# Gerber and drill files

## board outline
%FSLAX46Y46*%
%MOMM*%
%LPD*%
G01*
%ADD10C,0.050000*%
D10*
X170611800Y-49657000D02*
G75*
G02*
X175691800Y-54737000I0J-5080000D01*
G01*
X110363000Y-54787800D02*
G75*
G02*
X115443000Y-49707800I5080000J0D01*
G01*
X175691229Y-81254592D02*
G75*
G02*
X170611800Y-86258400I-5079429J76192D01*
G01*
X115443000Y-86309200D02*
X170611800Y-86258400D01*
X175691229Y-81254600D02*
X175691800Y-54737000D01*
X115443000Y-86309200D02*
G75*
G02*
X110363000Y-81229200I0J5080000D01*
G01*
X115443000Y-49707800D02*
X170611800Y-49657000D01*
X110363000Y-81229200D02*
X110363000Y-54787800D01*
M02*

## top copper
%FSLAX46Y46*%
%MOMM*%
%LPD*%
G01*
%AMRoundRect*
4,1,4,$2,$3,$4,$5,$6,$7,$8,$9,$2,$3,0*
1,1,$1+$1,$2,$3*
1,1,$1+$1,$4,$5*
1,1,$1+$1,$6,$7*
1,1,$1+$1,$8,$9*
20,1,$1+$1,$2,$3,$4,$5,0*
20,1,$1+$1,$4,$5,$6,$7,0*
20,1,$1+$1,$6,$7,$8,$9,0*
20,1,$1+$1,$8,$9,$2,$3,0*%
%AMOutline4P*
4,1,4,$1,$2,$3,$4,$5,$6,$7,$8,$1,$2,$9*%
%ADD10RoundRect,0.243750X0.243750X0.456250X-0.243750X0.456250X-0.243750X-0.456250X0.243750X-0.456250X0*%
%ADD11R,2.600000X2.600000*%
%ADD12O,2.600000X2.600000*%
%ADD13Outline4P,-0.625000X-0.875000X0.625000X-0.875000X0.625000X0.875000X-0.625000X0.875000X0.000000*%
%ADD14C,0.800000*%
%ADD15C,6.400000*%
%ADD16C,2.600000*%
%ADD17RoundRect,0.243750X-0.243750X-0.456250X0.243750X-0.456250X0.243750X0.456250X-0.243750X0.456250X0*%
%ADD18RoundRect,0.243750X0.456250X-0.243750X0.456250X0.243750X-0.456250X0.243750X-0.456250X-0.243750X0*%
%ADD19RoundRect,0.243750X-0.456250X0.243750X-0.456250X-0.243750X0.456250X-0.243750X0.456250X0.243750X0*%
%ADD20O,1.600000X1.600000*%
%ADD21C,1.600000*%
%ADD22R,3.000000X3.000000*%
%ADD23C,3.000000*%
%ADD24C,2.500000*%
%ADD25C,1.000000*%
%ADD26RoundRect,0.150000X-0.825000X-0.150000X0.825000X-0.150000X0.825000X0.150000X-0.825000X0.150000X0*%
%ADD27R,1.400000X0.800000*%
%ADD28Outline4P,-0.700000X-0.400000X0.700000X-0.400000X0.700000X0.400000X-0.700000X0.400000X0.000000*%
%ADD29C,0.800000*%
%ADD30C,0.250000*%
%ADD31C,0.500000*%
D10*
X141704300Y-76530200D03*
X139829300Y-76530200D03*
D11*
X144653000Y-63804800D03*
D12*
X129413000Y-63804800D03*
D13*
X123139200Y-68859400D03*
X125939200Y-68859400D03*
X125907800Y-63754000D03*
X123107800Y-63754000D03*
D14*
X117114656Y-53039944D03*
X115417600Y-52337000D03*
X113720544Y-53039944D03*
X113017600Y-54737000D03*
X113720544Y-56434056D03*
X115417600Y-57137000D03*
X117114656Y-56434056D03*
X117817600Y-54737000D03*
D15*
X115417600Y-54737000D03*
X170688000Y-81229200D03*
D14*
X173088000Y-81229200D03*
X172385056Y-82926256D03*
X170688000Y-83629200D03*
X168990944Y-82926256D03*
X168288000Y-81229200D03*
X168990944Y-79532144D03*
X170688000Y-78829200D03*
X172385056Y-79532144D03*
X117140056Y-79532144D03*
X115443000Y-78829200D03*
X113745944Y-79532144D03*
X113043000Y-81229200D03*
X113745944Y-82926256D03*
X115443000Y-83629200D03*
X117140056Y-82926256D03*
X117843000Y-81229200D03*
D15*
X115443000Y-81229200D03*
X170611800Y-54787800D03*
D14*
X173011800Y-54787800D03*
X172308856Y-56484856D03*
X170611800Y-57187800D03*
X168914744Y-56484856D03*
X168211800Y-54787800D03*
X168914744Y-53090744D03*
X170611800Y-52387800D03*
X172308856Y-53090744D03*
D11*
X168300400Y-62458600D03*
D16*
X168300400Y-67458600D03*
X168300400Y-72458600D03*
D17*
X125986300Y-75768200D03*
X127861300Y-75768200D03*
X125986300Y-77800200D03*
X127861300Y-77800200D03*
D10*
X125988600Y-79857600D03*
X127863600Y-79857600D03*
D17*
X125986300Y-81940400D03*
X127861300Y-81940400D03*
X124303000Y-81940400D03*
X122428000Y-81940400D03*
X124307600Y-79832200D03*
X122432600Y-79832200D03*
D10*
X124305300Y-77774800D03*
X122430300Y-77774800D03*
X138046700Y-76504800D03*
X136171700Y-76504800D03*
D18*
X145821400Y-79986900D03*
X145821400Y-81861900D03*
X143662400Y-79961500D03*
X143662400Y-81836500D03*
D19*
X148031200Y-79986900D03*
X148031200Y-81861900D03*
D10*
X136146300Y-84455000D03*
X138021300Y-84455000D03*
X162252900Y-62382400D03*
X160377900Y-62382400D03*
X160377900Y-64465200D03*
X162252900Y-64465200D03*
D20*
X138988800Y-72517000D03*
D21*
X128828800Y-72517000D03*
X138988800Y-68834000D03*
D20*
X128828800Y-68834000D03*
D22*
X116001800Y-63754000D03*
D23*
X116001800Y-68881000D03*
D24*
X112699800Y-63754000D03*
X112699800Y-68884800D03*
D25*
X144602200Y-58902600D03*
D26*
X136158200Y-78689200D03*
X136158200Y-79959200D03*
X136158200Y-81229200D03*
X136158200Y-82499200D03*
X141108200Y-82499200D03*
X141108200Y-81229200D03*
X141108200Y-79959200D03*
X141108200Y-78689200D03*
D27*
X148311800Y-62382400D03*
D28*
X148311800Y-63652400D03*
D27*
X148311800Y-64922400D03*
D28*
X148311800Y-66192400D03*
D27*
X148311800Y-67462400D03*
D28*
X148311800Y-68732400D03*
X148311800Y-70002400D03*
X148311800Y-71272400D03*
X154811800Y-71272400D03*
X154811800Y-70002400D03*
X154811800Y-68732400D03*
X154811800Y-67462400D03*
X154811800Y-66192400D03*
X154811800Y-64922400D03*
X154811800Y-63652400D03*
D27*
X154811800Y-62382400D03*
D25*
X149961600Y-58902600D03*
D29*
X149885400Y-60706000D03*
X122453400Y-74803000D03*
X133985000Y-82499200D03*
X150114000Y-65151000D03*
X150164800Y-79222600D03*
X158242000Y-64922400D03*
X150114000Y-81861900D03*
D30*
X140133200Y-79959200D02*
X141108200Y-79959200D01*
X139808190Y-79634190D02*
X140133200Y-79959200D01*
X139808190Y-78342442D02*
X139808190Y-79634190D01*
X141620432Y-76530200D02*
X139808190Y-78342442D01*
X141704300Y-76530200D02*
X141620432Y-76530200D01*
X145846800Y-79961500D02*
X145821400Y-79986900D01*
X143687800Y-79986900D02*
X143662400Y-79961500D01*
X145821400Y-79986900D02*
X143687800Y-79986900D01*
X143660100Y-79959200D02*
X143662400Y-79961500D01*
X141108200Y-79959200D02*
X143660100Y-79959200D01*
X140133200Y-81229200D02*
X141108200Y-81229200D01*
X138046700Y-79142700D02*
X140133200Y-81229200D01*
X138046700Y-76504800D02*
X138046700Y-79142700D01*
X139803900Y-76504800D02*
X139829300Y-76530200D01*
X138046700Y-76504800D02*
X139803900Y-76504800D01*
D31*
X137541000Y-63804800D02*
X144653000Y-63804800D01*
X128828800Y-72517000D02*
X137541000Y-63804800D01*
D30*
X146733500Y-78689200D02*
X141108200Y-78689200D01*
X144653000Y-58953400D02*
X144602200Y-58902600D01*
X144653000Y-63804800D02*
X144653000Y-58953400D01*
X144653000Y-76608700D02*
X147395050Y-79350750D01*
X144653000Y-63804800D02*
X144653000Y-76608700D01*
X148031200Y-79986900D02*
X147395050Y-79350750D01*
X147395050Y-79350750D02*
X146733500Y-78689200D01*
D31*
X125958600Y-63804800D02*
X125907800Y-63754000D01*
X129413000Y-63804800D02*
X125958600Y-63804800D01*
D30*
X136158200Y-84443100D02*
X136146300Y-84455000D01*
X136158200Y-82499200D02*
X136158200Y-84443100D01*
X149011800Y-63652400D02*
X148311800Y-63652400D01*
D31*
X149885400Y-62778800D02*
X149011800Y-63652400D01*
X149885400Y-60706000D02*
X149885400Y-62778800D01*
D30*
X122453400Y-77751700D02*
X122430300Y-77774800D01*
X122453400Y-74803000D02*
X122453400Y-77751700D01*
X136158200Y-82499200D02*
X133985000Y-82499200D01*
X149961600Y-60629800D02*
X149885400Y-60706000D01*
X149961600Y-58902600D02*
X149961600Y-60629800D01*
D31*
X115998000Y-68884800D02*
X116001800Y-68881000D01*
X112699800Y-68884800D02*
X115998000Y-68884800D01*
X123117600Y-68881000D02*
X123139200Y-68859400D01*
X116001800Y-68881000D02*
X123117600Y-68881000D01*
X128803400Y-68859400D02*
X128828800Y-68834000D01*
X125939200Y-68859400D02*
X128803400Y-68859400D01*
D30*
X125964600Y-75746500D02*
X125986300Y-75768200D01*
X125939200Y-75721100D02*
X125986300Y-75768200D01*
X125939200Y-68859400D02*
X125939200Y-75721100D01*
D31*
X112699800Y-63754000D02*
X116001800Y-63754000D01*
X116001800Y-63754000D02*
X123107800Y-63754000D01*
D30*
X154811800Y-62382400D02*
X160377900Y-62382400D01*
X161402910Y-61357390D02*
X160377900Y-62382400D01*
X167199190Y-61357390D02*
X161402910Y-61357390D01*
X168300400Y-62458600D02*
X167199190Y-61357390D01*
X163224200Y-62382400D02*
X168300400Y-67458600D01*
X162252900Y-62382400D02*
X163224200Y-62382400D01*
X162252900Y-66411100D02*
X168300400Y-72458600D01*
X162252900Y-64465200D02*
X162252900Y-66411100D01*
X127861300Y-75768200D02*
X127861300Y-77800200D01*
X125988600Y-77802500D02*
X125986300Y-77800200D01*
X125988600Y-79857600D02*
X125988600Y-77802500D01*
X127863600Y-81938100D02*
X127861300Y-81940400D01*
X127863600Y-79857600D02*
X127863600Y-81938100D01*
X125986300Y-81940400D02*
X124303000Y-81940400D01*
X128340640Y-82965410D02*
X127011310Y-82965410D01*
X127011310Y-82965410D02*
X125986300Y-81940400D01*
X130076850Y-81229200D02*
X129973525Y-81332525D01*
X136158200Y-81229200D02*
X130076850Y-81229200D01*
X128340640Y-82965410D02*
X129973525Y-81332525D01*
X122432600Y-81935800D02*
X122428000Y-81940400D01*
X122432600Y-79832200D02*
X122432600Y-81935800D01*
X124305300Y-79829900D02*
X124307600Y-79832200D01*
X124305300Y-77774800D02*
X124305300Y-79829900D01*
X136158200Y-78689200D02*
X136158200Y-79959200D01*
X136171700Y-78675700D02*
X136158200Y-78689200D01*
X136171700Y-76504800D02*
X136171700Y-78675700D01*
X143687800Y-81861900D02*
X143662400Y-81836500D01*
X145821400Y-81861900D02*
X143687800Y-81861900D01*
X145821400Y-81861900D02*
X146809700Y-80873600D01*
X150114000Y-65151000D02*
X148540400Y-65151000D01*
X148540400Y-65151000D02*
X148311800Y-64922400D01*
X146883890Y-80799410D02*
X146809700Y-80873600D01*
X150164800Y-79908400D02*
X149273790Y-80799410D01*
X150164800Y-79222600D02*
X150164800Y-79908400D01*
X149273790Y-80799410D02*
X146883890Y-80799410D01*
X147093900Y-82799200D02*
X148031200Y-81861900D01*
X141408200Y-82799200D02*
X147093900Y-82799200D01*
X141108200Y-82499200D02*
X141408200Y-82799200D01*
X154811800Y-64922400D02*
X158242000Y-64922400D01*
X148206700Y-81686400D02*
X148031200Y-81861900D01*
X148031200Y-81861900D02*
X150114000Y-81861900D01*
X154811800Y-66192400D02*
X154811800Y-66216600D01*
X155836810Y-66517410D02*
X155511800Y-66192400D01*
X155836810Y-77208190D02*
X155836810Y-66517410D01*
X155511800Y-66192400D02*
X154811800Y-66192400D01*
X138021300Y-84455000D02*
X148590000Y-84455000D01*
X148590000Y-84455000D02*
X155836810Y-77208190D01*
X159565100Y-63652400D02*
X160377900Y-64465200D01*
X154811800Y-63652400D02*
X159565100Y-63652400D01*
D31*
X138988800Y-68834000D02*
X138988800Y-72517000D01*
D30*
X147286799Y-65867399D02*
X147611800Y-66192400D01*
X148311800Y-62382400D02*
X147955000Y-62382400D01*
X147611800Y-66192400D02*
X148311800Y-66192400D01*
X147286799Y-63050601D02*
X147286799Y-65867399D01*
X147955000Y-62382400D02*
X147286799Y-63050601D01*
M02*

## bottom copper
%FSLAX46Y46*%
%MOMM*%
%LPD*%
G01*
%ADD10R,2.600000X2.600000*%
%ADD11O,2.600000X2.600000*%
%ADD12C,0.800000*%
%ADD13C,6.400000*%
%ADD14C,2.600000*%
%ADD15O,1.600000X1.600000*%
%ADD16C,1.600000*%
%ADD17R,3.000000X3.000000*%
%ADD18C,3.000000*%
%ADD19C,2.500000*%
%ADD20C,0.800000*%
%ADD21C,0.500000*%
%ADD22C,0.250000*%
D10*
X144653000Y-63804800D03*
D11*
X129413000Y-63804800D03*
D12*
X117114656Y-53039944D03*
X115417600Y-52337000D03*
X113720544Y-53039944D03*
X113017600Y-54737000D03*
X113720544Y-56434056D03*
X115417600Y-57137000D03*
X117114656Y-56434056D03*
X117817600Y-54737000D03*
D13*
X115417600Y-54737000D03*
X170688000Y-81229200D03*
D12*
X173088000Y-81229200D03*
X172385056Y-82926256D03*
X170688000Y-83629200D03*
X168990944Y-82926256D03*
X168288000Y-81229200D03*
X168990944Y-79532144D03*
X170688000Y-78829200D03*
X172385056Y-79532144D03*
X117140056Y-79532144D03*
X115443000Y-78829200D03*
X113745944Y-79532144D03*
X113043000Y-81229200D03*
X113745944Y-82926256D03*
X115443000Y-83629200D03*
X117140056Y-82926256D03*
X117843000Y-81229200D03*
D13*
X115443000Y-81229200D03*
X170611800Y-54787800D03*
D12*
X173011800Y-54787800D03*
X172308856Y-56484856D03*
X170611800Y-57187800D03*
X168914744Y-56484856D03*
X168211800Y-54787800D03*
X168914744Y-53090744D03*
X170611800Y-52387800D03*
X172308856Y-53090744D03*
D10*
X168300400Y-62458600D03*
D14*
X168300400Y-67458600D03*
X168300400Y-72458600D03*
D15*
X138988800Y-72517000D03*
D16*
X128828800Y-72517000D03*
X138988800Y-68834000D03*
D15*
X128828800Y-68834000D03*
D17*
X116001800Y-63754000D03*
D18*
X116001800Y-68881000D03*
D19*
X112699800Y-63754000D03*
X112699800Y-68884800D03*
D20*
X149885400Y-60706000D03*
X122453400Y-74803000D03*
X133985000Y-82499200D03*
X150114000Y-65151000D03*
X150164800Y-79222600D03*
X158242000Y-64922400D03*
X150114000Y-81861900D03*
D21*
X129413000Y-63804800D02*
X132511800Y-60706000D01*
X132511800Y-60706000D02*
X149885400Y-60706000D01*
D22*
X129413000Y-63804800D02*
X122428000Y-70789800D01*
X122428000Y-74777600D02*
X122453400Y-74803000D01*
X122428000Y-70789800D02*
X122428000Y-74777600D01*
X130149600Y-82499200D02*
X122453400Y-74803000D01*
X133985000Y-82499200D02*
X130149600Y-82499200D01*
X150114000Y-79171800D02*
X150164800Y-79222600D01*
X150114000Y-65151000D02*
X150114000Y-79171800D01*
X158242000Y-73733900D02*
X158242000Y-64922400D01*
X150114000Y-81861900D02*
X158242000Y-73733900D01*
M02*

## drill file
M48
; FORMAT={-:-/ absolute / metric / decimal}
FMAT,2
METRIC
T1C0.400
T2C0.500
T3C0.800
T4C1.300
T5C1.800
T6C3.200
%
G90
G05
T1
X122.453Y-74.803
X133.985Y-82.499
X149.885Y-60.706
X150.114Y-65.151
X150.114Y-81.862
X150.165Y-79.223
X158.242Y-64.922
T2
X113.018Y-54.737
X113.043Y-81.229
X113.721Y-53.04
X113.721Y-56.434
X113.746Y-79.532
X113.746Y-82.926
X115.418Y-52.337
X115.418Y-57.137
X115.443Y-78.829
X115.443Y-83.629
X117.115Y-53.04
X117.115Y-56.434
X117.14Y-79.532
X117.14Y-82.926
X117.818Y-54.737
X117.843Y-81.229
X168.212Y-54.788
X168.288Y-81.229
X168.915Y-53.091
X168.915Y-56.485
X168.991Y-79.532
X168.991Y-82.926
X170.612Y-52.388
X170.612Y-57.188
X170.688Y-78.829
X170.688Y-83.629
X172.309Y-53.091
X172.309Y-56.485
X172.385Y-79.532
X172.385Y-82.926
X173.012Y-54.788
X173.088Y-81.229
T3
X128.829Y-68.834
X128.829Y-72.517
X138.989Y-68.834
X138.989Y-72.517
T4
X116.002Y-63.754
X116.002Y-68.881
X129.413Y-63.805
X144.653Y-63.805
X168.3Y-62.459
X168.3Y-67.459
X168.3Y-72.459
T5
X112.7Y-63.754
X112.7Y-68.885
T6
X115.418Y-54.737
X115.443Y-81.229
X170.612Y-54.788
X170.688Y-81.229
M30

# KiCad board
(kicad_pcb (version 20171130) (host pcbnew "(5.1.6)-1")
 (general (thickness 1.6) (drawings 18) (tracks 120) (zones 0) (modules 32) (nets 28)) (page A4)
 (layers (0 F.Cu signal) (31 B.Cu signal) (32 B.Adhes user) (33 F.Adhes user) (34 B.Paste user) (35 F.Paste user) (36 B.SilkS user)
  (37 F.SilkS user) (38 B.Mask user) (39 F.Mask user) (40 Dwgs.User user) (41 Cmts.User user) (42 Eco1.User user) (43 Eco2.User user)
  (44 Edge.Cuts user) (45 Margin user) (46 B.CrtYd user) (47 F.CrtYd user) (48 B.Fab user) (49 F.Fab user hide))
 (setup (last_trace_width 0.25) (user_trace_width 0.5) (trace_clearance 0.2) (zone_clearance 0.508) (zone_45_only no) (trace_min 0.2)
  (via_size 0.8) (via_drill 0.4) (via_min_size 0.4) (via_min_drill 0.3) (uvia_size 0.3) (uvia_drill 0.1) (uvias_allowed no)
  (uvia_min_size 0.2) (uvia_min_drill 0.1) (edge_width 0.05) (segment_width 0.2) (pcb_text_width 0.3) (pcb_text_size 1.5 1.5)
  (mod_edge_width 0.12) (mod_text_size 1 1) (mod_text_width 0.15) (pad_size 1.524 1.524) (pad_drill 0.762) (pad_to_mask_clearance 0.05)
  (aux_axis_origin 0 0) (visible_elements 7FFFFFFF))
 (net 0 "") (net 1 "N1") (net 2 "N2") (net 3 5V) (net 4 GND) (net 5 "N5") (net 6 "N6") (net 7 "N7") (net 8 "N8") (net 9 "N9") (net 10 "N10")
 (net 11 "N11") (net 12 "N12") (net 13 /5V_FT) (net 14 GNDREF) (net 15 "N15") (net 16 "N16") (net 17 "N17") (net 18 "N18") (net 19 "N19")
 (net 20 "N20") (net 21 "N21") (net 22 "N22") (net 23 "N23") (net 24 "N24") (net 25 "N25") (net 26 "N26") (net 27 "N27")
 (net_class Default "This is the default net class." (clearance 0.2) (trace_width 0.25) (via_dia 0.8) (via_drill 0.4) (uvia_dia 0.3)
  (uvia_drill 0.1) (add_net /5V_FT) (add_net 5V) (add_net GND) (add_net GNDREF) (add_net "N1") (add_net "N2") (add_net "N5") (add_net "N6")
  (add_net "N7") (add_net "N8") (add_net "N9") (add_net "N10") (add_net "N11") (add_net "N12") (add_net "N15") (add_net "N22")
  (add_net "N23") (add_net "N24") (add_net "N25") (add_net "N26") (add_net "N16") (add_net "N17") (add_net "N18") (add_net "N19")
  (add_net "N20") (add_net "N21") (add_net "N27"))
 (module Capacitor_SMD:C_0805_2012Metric (layer F.Cu) (at 140.7668 76.5302 180)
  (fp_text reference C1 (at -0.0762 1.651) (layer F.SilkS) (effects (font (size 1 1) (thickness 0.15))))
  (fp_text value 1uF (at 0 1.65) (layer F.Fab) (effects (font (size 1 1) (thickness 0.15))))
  (pad 1 smd roundrect (at -0.9375 0 180) (size 0.975 1.4) (layers F.Cu F.Paste F.Mask) (roundrect_rratio 0.25) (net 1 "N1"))
  (pad 2 smd roundrect (at 0.9375 0 180) (size 0.975 1.4) (layers F.Cu F.Paste F.Mask) (roundrect_rratio 0.25) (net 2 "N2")))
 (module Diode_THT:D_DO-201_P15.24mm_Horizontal (layer F.Cu) (at 144.653 63.8048 180)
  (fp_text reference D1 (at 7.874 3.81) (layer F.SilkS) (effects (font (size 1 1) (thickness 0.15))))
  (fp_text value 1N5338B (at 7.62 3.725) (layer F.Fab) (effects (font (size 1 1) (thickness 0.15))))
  (pad 1 thru_hole rect (at 0 0 180) (size 2.6 2.6) (drill 1.3) (layers *.Cu *.Mask) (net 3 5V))
  (pad 2 thru_hole oval (at 15.24 0 180) (size 2.6 2.6) (drill 1.3) (layers *.Cu *.Mask) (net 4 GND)))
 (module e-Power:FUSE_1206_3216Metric (layer F.Cu) (at 124.5392 68.8594)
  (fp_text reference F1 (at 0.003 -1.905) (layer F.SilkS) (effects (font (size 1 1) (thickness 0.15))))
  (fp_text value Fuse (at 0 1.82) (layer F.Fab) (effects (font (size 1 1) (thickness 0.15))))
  (pad 1 smd trapezoid (at -1.4 0) (size 1.25 1.75) (layers F.Cu F.Paste F.Mask) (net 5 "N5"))
  (pad 2 smd trapezoid (at 1.4 0) (size 1.25 1.75) (layers F.Cu F.Paste F.Mask) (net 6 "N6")))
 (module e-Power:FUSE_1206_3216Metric (layer F.Cu) (at 124.5078 63.754)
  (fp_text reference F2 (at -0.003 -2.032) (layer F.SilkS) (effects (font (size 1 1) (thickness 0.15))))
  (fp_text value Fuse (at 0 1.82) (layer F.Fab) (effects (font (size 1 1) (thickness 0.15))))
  (pad 2 smd trapezoid (at 1.4 0) (size 1.25 1.75) (layers F.Cu F.Paste F.Mask) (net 4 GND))
  (pad 1 smd trapezoid (at -1.4 0) (size 1.25 1.75) (layers F.Cu F.Paste F.Mask) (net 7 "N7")))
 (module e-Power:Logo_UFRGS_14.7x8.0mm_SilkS (layer F.Cu) (at 159.3596 81.2546)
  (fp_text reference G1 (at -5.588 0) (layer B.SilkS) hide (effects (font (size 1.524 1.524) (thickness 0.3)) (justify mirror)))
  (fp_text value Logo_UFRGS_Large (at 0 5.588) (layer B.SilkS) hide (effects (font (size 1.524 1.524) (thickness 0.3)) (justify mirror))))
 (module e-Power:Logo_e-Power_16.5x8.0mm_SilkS (layer F.Cu) (at 158.1912 54.7878)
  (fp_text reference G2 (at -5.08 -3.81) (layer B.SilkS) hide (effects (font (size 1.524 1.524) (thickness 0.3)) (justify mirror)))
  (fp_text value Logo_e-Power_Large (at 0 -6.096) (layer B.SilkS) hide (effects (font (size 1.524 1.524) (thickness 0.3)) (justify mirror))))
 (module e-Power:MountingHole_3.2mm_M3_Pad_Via (layer F.Cu) (at 115.4176 54.737)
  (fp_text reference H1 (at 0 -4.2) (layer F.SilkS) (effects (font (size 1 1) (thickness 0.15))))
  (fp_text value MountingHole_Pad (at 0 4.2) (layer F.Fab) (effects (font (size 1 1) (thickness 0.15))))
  (pad 1 thru_hole circle (at 1.697056 -1.697056) (size 0.8 0.8) (drill 0.5) (layers *.Cu *.Mask) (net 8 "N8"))
  (pad 1 thru_hole circle (at 0 -2.4) (size 0.8 0.8) (drill 0.5) (layers *.Cu *.Mask) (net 8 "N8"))
  (pad 1 thru_hole circle (at -1.697056 -1.697056) (size 0.8 0.8) (drill 0.5) (layers *.Cu *.Mask) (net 8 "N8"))
  (pad 1 thru_hole circle (at -2.4 0) (size 0.8 0.8) (drill 0.5) (layers *.Cu *.Mask) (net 8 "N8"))
  (pad 1 thru_hole circle (at -1.697056 1.697056) (size 0.8 0.8) (drill 0.5) (layers *.Cu *.Mask) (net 8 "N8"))
  (pad 1 thru_hole circle (at 0 2.4) (size 0.8 0.8) (drill 0.5) (layers *.Cu *.Mask) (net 8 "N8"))
  (pad 1 thru_hole circle (at 1.697056 1.697056) (size 0.8 0.8) (drill 0.5) (layers *.Cu *.Mask) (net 8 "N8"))
  (pad 1 thru_hole circle (at 2.4 0) (size 0.8 0.8) (drill 0.5) (layers *.Cu *.Mask) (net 8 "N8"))
  (pad 1 thru_hole circle (at 0 0) (size 6.4 6.4) (drill 3.2) (layers *.Cu *.Mask) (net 8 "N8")))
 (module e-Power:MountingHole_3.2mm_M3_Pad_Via (layer F.Cu) (at 170.688 81.2292)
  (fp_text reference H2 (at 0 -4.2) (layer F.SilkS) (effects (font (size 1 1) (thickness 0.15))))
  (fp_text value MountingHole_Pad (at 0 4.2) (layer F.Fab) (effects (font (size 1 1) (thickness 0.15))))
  (pad 1 thru_hole circle (at 0 0) (size 6.4 6.4) (drill 3.2) (layers *.Cu *.Mask) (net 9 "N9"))
  (pad 1 thru_hole circle (at 2.4 0) (size 0.8 0.8) (drill 0.5) (layers *.Cu *.Mask) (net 9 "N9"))
  (pad 1 thru_hole circle (at 1.697056 1.697056) (size 0.8 0.8) (drill 0.5) (layers *.Cu *.Mask) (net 9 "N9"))
  (pad 1 thru_hole circle (at 0 2.4) (size 0.8 0.8) (drill 0.5) (layers *.Cu *.Mask) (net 9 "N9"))
  (pad 1 thru_hole circle (at -1.697056 1.697056) (size 0.8 0.8) (drill 0.5) (layers *.Cu *.Mask) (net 9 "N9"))
  (pad 1 thru_hole circle (at -2.4 0) (size 0.8 0.8) (drill 0.5) (layers *.Cu *.Mask) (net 9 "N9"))
  (pad 1 thru_hole circle (at -1.697056 -1.697056) (size 0.8 0.8) (drill 0.5) (layers *.Cu *.Mask) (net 9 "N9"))
  (pad 1 thru_hole circle (at 0 -2.4) (size 0.8 0.8) (drill 0.5) (layers *.Cu *.Mask) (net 9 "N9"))
  (pad 1 thru_hole circle (at 1.697056 -1.697056) (size 0.8 0.8) (drill 0.5) (layers *.Cu *.Mask) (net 9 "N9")))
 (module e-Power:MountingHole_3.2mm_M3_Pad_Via (layer F.Cu) (at 115.443 81.2292)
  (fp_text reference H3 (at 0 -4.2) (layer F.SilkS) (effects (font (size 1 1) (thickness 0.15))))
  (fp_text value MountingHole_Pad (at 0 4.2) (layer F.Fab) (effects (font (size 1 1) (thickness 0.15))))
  (pad 1 thru_hole circle (at 1.697056 -1.697056) (size 0.8 0.8) (drill 0.5) (layers *.Cu *.Mask) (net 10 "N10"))
  (pad 1 thru_hole circle (at 0 -2.4) (size 0.8 0.8) (drill 0.5) (layers *.Cu *.Mask) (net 10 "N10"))
  (pad 1 thru_hole circle (at -1.697056 -1.697056) (size 0.8 0.8) (drill 0.5) (layers *.Cu *.Mask) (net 10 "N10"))
  (pad 1 thru_hole circle (at -2.4 0) (size 0.8 0.8) (drill 0.5) (layers *.Cu *.Mask) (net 10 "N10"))
  (pad 1 thru_hole circle (at -1.697056 1.697056) (size 0.8 0.8) (drill 0.5) (layers *.Cu *.Mask) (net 10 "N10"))
  (pad 1 thru_hole circle (at 0 2.4) (size 0.8 0.8) (drill 0.5) (layers *.Cu *.Mask) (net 10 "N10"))
  (pad 1 thru_hole circle (at 1.697056 1.697056) (size 0.8 0.8) (drill 0.5) (layers *.Cu *.Mask) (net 10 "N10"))
  (pad 1 thru_hole circle (at 2.4 0) (size 0.8 0.8) (drill 0.5) (layers *.Cu *.Mask) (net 10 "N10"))
  (pad 1 thru_hole circle (at 0 0) (size 6.4 6.4) (drill 3.2) (layers *.Cu *.Mask) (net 10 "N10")))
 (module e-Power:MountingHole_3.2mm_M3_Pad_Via (layer F.Cu) (at 170.6118 54.7878)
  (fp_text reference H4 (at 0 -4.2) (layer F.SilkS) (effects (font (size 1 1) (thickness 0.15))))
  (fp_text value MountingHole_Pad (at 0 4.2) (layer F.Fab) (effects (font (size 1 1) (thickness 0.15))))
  (pad 1 thru_hole circle (at 0 0) (size 6.4 6.4) (drill 3.2) (layers *.Cu *.Mask) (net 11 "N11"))
  (pad 1 thru_hole circle (at 2.4 0) (size 0.8 0.8) (drill 0.5) (layers *.Cu *.Mask) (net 11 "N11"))
  (pad 1 thru_hole circle (at 1.697056 1.697056) (size 0.8 0.8) (drill 0.5) (layers *.Cu *.Mask) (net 11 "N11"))
  (pad 1 thru_hole circle (at 0 2.4) (size 0.8 0.8) (drill 0.5) (layers *.Cu *.Mask) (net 11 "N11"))
  (pad 1 thru_hole circle (at -1.697056 1.697056) (size 0.8 0.8) (drill 0.5) (layers *.Cu *.Mask) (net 11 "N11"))
  (pad 1 thru_hole circle (at -2.4 0) (size 0.8 0.8) (drill 0.5) (layers *.Cu *.Mask) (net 11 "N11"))
  (pad 1 thru_hole circle (at -1.697056 -1.697056) (size 0.8 0.8) (drill 0.5) (layers *.Cu *.Mask) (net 11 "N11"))
  (pad 1 thru_hole circle (at 0 -2.4) (size 0.8 0.8) (drill 0.5) (layers *.Cu *.Mask) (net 11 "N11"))
  (pad 1 thru_hole circle (at 1.697056 -1.697056) (size 0.8 0.8) (drill 0.5) (layers *.Cu *.Mask) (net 11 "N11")))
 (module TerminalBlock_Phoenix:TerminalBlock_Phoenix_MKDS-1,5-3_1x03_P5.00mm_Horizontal (layer F.Cu) (at 168.3004 62.4586 270)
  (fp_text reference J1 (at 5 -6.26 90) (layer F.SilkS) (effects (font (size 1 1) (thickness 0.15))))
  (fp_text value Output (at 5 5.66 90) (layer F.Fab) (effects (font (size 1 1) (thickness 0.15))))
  (pad 1 thru_hole rect (at 0 0 270) (size 2.6 2.6) (drill 1.3) (layers *.Cu *.Mask) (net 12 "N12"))
  (pad 2 thru_hole circle (at 5 0 270) (size 2.6 2.6) (drill 1.3) (layers *.Cu *.Mask) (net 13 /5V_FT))
  (pad 3 thru_hole circle (at 10 0 270) (size 2.6 2.6) (drill 1.3) (layers *.Cu *.Mask) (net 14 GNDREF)))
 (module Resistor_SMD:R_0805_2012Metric (layer F.Cu) (at 126.9238 75.7682)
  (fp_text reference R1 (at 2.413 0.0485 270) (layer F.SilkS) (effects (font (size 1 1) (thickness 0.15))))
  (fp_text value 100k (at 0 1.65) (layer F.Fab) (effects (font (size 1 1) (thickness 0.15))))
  (pad 1 smd roundrect (at -0.9375 0) (size 0.975 1.4) (layers F.Cu F.Paste F.Mask) (roundrect_rratio 0.25) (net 6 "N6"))
  (pad 2 smd roundrect (at 0.9375 0) (size 0.975 1.4) (layers F.Cu F.Paste F.Mask) (roundrect_rratio 0.25) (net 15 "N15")))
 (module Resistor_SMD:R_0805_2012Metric (layer F.Cu) (at 126.9238 77.8002)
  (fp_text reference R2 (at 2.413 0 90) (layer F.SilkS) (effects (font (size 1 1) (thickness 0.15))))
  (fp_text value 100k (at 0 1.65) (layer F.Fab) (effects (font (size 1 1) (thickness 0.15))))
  (pad 1 smd roundrect (at -0.9375 0) (size 0.975 1.4) (layers F.Cu F.Paste F.Mask) (roundrect_rratio 0.25) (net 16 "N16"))
  (pad 2 smd roundrect (at 0.9375 0) (size 0.975 1.4) (layers F.Cu F.Paste F.Mask) (roundrect_rratio 0.25) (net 15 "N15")))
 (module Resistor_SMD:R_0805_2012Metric (layer F.Cu) (at 126.9261 79.8576 180)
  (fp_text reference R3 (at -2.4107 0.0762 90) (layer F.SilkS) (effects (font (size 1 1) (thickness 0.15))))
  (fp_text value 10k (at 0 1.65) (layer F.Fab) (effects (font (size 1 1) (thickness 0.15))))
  (pad 2 smd roundrect (at 0.9375 0 180) (size 0.975 1.4) (layers F.Cu F.Paste F.Mask) (roundrect_rratio 0.25) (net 16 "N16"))
  (pad 1 smd roundrect (at -0.9375 0 180) (size 0.975 1.4) (layers F.Cu F.Paste F.Mask) (roundrect_rratio 0.25) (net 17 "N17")))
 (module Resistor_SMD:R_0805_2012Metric (layer F.Cu) (at 126.9238 81.9404)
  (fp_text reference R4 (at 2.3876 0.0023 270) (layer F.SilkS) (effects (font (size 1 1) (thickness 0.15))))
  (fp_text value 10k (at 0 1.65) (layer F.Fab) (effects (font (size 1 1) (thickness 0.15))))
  (pad 1 smd roundrect (at -0.9375 0) (size 0.975 1.4) (layers F.Cu F.Paste F.Mask) (roundrect_rratio 0.25) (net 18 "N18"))
  (pad 2 smd roundrect (at 0.9375 0) (size 0.975 1.4) (layers F.Cu F.Paste F.Mask) (roundrect_rratio 0.25) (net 17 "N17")))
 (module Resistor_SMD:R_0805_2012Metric (layer F.Cu) (at 123.3655 81.9404)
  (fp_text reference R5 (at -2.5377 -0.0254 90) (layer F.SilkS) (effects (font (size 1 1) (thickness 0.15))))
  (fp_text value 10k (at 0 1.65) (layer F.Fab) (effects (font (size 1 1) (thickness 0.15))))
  (pad 2 smd roundrect (at 0.9375 0) (size 0.975 1.4) (layers F.Cu F.Paste F.Mask) (roundrect_rratio 0.25) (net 18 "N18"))
  (pad 1 smd roundrect (at -0.9375 0) (size 0.975 1.4) (layers F.Cu F.Paste F.Mask) (roundrect_rratio 0.25) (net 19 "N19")))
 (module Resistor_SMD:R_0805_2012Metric (layer F.Cu) (at 123.3701 79.8322)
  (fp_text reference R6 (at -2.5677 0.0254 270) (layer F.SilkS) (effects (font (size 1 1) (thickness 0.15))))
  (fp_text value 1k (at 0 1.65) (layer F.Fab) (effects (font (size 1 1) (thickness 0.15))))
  (pad 2 smd roundrect (at 0.9375 0) (size 0.975 1.4) (layers F.Cu F.Paste F.Mask) (roundrect_rratio 0.25) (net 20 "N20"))
  (pad 1 smd roundrect (at -0.9375 0) (size 0.975 1.4) (layers F.Cu F.Paste F.Mask) (roundrect_rratio 0.25) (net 19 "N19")))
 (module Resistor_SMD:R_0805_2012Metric (layer F.Cu) (at 123.3678 77.7748 180)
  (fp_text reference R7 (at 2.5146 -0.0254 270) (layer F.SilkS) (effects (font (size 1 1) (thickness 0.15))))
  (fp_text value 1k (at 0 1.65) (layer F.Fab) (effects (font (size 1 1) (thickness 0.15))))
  (pad 1 smd roundrect (at -0.9375 0 180) (size 0.975 1.4) (layers F.Cu F.Paste F.Mask) (roundrect_rratio 0.25) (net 20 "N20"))
  (pad 2 smd roundrect (at 0.9375 0 180) (size 0.975 1.4) (layers F.Cu F.Paste F.Mask) (roundrect_rratio 0.25) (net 4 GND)))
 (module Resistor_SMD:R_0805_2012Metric (layer F.Cu) (at 137.1092 76.5048 180)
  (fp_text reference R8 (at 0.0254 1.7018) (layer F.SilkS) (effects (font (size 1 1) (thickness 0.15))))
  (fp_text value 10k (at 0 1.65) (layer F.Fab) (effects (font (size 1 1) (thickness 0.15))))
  (pad 1 smd roundrect (at -0.9375 0 180) (size 0.975 1.4) (layers F.Cu F.Paste F.Mask) (roundrect_rratio 0.25) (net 2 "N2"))
  (pad 2 smd roundrect (at 0.9375 0 180) (size 0.975 1.4) (layers F.Cu F.Paste F.Mask) (roundrect_rratio 0.25) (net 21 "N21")))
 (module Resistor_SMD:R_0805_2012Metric (layer F.Cu) (at 145.8214 80.9244 90)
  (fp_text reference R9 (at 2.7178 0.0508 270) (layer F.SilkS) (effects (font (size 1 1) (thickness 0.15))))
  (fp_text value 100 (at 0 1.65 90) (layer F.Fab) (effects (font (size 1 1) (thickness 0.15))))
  (pad 2 smd roundrect (at 0.9375 0 90) (size 0.975 1.4) (layers F.Cu F.Paste F.Mask) (roundrect_rratio 0.25) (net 1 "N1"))
  (pad 1 smd roundrect (at -0.9375 0 90) (size 0.975 1.4) (layers F.Cu F.Paste F.Mask) (roundrect_rratio 0.25) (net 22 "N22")))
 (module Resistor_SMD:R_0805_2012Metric (layer F.Cu) (at 143.6624 80.899 90)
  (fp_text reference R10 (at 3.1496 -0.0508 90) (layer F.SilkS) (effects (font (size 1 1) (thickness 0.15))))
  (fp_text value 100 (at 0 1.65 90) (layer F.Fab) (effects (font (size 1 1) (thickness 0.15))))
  (pad 2 smd roundrect (at 0.9375 0 90) (size 0.975 1.4) (layers F.Cu F.Paste F.Mask) (roundrect_rratio 0.25) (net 1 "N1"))
  (pad 1 smd roundrect (at -0.9375 0 90) (size 0.975 1.4) (layers F.Cu F.Paste F.Mask) (roundrect_rratio 0.25) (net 22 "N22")))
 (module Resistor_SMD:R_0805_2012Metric (layer F.Cu) (at 148.0312 80.9244 270)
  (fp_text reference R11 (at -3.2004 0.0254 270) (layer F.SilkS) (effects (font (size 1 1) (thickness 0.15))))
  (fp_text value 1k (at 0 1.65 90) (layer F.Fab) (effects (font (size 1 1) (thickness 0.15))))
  (pad 1 smd roundrect (at -0.9375 0 270) (size 0.975 1.4) (layers F.Cu F.Paste F.Mask) (roundrect_rratio 0.25) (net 3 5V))
  (pad 2 smd roundrect (at 0.9375 0 270) (size 0.975 1.4) (layers F.Cu F.Paste F.Mask) (roundrect_rratio 0.25) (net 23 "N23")))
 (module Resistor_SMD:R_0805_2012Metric (layer F.Cu) (at 137.0838 84.455 180)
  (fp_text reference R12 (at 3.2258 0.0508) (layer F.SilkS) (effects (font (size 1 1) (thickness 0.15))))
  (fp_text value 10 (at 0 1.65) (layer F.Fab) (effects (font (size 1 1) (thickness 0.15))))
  (pad 2 smd roundrect (at 0.9375 0 180) (size 0.975 1.4) (layers F.Cu F.Paste F.Mask) (roundrect_rratio 0.25) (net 4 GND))
  (pad 1 smd roundrect (at -0.9375 0 180) (size 0.975 1.4) (layers F.Cu F.Paste F.Mask) (roundrect_rratio 0.25) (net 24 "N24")))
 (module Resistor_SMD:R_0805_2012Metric (layer F.Cu) (at 161.3154 62.3824 180)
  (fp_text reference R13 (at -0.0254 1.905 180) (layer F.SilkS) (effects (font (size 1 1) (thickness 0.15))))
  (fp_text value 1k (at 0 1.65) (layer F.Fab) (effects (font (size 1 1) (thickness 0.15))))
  (pad 1 smd roundrect (at -0.9375 0 180) (size 0.975 1.4) (layers F.Cu F.Paste F.Mask) (roundrect_rratio 0.25) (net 13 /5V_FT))
  (pad 2 smd roundrect (at 0.9375 0 180) (size 0.975 1.4) (layers F.Cu F.Paste F.Mask) (roundrect_rratio 0.25) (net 12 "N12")))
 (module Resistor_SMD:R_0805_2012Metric (layer F.Cu) (at 161.3154 64.4652 180)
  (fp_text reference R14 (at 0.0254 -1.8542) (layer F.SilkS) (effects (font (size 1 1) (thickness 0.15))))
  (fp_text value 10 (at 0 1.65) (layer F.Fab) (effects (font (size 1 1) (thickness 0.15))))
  (pad 2 smd roundrect (at 0.9375 0 180) (size 0.975 1.4) (layers F.Cu F.Paste F.Mask) (roundrect_rratio 0.25) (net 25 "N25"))
  (pad 1 smd roundrect (at -0.9375 0 180) (size 0.975 1.4) (layers F.Cu F.Paste F.Mask) (roundrect_rratio 0.25) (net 14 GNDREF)))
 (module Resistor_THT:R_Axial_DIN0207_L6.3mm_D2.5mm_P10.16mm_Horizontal (layer F.Cu) (at 128.8288 72.517)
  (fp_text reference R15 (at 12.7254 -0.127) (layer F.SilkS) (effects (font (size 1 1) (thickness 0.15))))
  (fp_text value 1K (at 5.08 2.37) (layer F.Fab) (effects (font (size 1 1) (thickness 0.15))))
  (pad 2 thru_hole oval (at 10.16 0) (size 1.6 1.6) (drill 0.8) (layers *.Cu *.Mask) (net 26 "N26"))
  (pad 1 thru_hole circle (at 0 0) (size 1.6 1.6) (drill 0.8) (layers *.Cu *.Mask) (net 3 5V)))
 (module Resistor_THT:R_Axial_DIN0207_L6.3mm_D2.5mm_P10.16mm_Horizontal (layer F.Cu) (at 138.9888 68.834 180)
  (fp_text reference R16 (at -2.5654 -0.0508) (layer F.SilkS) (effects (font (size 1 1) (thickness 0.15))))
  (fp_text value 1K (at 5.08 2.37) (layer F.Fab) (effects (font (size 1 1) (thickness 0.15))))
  (pad 1 thru_hole circle (at 0 0 180) (size 1.6 1.6) (drill 0.8) (layers *.Cu *.Mask) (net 26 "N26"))
  (pad 2 thru_hole oval (at 10.16 0 180) (size 1.6 1.6) (drill 0.8) (layers *.Cu *.Mask) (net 6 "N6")))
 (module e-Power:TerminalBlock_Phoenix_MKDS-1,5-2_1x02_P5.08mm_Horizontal (layer F.Cu) (at 116.0018 63.754 270)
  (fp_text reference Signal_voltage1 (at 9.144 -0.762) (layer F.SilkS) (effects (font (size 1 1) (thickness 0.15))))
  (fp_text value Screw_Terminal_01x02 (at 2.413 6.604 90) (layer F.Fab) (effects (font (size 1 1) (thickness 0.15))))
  (pad 1 thru_hole rect (at 0 0 270) (size 3 3) (drill 1.3) (layers *.Cu *.Mask) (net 7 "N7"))
  (pad 2 thru_hole circle (at 5.127 0 270) (size 3 3) (drill 1.3) (layers *.Cu *.Mask) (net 5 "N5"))
  (pad 1 thru_hole circle (at 0 3.302 270) (size 2.5 2.5) (drill 1.8) (layers *.Cu *.Mask) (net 7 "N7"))
  (pad 2 thru_hole circle (at 5.1308 3.302 270) (size 2.5 2.5) (drill 1.8) (layers *.Cu *.Mask) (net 5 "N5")))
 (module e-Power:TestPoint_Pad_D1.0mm (layer F.Cu) (at 144.6022 58.9026)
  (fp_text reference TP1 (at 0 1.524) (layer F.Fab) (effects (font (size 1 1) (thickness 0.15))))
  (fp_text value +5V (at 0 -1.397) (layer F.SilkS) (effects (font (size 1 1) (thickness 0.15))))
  (pad 1 smd circle (at 0 0) (size 1 1) (layers F.Cu F.Mask) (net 3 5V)))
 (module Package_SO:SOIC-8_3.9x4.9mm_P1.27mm (layer F.Cu) (at 138.6332 80.5942)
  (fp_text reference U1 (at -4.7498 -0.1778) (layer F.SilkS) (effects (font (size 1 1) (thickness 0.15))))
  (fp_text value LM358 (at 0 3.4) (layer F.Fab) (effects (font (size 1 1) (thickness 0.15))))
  (pad 1 smd roundrect (at -2.475 -1.905) (size 1.95 0.6) (layers F.Cu F.Paste F.Mask) (roundrect_rratio 0.25) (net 21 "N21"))
  (pad 2 smd roundrect (at -2.475 -0.635) (size 1.95 0.6) (layers F.Cu F.Paste F.Mask) (roundrect_rratio 0.25) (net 21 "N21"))
  (pad 3 smd roundrect (at -2.475 0.635) (size 1.95 0.6) (layers F.Cu F.Paste F.Mask) (roundrect_rratio 0.25) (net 18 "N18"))
  (pad 4 smd roundrect (at -2.475 1.905) (size 1.95 0.6) (layers F.Cu F.Paste F.Mask) (roundrect_rratio 0.25) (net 4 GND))
  (pad 5 smd roundrect (at 2.475 1.905) (size 1.95 0.6) (layers F.Cu F.Paste F.Mask) (roundrect_rratio 0.25) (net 23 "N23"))
  (pad 6 smd roundrect (at 2.475 0.635) (size 1.95 0.6) (layers F.Cu F.Paste F.Mask) (roundrect_rratio 0.25) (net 2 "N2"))
  (pad 7 smd roundrect (at 2.475 -0.635) (size 1.95 0.6) (layers F.Cu F.Paste F.Mask) (roundrect_rratio 0.25) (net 1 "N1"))
  (pad 8 smd roundrect (at 2.475 -1.905) (size 1.95 0.6) (layers F.Cu F.Paste F.Mask) (roundrect_rratio 0.25) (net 3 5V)))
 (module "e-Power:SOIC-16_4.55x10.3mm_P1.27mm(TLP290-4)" (layer F.Cu) (at 151.5618 66.8274)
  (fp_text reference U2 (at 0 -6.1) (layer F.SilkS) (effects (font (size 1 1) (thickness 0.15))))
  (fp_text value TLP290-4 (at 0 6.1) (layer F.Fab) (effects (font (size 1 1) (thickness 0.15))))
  (pad 1 smd rect (at -3.25 -4.445) (size 1.4 0.8) (layers F.Cu F.Paste F.Mask) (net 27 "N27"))
  (pad 2 smd trapezoid (at -3.25 -3.175) (size 1.4 0.8) (layers F.Cu F.Paste F.Mask) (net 4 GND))
  (pad 3 smd rect (at -3.25 -1.905) (size 1.4 0.8) (layers F.Cu F.Paste F.Mask) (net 22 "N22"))
  (pad 4 smd trapezoid (at -3.25 -0.635) (size 1.4 0.8) (layers F.Cu F.Paste F.Mask) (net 27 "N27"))
  (pad 5 smd rect (at -3.25 0.635) (size 1.4 0.8) (layers F.Cu F.Paste F.Mask))
  (pad 6 smd trapezoid (at -3.25 1.905) (size 1.4 0.8) (layers F.Cu F.Paste F.Mask))
  (pad 7 smd trapezoid (at -3.25 3.175) (size 1.4 0.8) (layers F.Cu F.Paste F.Mask))
  (pad 8 smd trapezoid (at -3.25 4.445) (size 1.4 0.8) (layers F.Cu F.Paste F.Mask))
  (pad 9 smd trapezoid (at 3.25 4.445) (size 1.4 0.8) (layers F.Cu F.Paste F.Mask))
  (pad 10 smd trapezoid (at 3.25 3.175) (size 1.4 0.8) (layers F.Cu F.Paste F.Mask))
  (pad 11 smd trapezoid (at 3.25 1.905) (size 1.4 0.8) (layers F.Cu F.Paste F.Mask))
  (pad 12 smd trapezoid (at 3.25 0.635) (size 1.4 0.8) (layers F.Cu F.Paste F.Mask))
  (pad 13 smd trapezoid (at 3.25 -0.635) (size 1.4 0.8) (layers F.Cu F.Paste F.Mask) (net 24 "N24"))
  (pad 14 smd trapezoid (at 3.25 -1.905) (size 1.4 0.8) (layers F.Cu F.Paste F.Mask) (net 23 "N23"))
  (pad 15 smd trapezoid (at 3.25 -3.175) (size 1.4 0.8) (layers F.Cu F.Paste F.Mask) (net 25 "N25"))
  (pad 16 smd rect (at 3.25 -4.445) (size 1.4 0.8) (layers F.Cu F.Paste F.Mask) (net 12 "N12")))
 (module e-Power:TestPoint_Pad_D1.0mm (layer F.Cu) (at 149.9616 58.9026)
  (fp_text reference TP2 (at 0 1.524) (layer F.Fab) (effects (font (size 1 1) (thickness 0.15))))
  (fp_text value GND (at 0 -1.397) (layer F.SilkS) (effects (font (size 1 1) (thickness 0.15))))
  (pad 1 smd circle (at 0 0) (size 1 1) (layers F.Cu F.Mask) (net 4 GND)))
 (gr_arc (start 170.6118 54.737) (end 175.6918 54.737) (angle -90) (layer Edge.Cuts) (width 0.05))
 (gr_arc (start 115.443 54.7878) (end 115.443 49.7078) (angle -90) (layer Edge.Cuts) (width 0.05))
 (gr_arc (start 170.6118 81.1784) (end 170.6118 86.2584) (angle -89.1406171) (layer Edge.Cuts) (width 0.05))
 (gr_line (start 115.443 86.3092) (end 170.6118 86.2584) (layer Edge.Cuts) (width 0.05))
 (gr_line (start 175.691229 81.2546) (end 175.6918 54.737) (layer Edge.Cuts) (width 0.05))
 (gr_arc (start 115.443 81.2292) (end 110.363 81.2292) (angle -90) (layer Edge.Cuts) (width 0.05))
 (gr_line (start 115.443 49.7078) (end 170.6118 49.657) (layer Edge.Cuts) (width 0.05))
 (gr_line (start 110.363 81.2292) (end 110.363 54.7878) (layer Edge.Cuts) (width 0.05))
 (segment (start 140.1332 79.9592) (end 141.1082 79.9592) (width 0.25) (layer F.Cu) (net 1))
 (segment (start 139.80819 79.63419) (end 140.1332 79.9592) (width 0.25) (layer F.Cu) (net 1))
 (segment (start 139.80819 78.342442) (end 139.80819 79.63419) (width 0.25) (layer F.Cu) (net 1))
 (segment (start 141.620432 76.5302) (end 139.80819 78.342442) (width 0.25) (layer F.Cu) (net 1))
 (segment (start 141.7043 76.5302) (end 141.620432 76.5302) (width 0.25) (layer F.Cu) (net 1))
 (segment (start 145.8468 79.9615) (end 145.8214 79.9869) (width 0.25) (layer F.Cu) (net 1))
 (segment (start 143.6878 79.9869) (end 143.6624 79.9615) (width 0.25) (layer F.Cu) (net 1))
 (segment (start 145.8214 79.9869) (end 143.6878 79.9869) (width 0.25) (layer F.Cu) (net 1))
 (segment (start 143.6601 79.9592) (end 143.6624 79.9615) (width 0.25) (layer F.Cu) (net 1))
 (segment (start 141.1082 79.9592) (end 143.6601 79.9592) (width 0.25) (layer F.Cu) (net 1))
 (segment (start 140.1332 81.2292) (end 141.1082 81.2292) (width 0.25) (layer F.Cu) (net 2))
 (segment (start 138.0467 79.1427) (end 140.1332 81.2292) (width 0.25) (layer F.Cu) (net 2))
 (segment (start 138.0467 76.5048) (end 138.0467 79.1427) (width 0.25) (layer F.Cu) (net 2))
 (segment (start 139.8039 76.5048) (end 139.8293 76.5302) (width 0.25) (layer F.Cu) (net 2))
 (segment (start 138.0467 76.5048) (end 139.8039 76.5048) (width 0.25) (layer F.Cu) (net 2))
 (segment (start 137.541 63.8048) (end 144.653 63.8048) (width 0.5) (layer F.Cu) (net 3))
 (segment (start 128.8288 72.517) (end 137.541 63.8048) (width 0.5) (layer F.Cu) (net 3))
 (segment (start 146.7335 78.6892) (end 141.1082 78.6892) (width 0.25) (layer F.Cu) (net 3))
 (segment (start 144.653 58.9534) (end 144.6022 58.9026) (width 0.25) (layer F.Cu) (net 3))
 (segment (start 144.653 63.8048) (end 144.653 58.9534) (width 0.25) (layer F.Cu) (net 3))
 (segment (start 144.653 76.6087) (end 147.39505 79.35075) (width 0.25) (layer F.Cu) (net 3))
 (segment (start 144.653 63.8048) (end 144.653 76.6087) (width 0.25) (layer F.Cu) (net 3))
 (segment (start 148.0312 79.9869) (end 147.39505 79.35075) (width 0.25) (layer F.Cu) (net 3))
 (segment (start 147.39505 79.35075) (end 146.7335 78.6892) (width 0.25) (layer F.Cu) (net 3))
 (segment (start 125.9586 63.8048) (end 125.9078 63.754) (width 0.5) (layer F.Cu) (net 4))
 (segment (start 129.413 63.8048) (end 125.9586 63.8048) (width 0.5) (layer F.Cu) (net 4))
 (segment (start 136.1582 84.4431) (end 136.1463 84.455) (width 0.25) (layer F.Cu) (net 4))
 (segment (start 136.1582 82.4992) (end 136.1582 84.4431) (width 0.25) (layer F.Cu) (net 4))
 (segment (start 129.413 63.8048) (end 132.5118 60.706) (width 0.5) (layer B.Cu) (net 4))
 (via (at 149.8854 60.706) (size 0.8) (drill 0.4) (layers F.Cu B.Cu) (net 4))
 (segment (start 132.5118 60.706) (end 149.8854 60.706) (width 0.5) (layer B.Cu) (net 4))
 (segment (start 149.0118 63.6524) (end 148.3118 63.6524) (width 0.25) (layer F.Cu) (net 4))
 (segment (start 149.8854 62.7788) (end 149.0118 63.6524) (width 0.5) (layer F.Cu) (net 4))
 (segment (start 149.8854 60.706) (end 149.8854 62.7788) (width 0.5) (layer F.Cu) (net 4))
 (segment (start 129.413 63.8048) (end 122.428 70.7898) (width 0.25) (layer B.Cu) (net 4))
 (via (at 122.4534 74.803) (size 0.8) (drill 0.4) (layers F.Cu B.Cu) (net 4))
 (segment (start 122.4534 77.7517) (end 122.4303 77.7748) (width 0.25) (layer F.Cu) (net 4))
 (segment (start 122.4534 74.803) (end 122.4534 77.7517) (width 0.25) (layer F.Cu) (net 4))
 (segment (start 136.1582 82.4992) (end 133.985 82.4992) (width 0.25) (layer F.Cu) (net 4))
 (via (at 133.985 82.4992) (size 0.8) (drill 0.4) (layers F.Cu B.Cu) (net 4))
 (segment (start 122.428 74.7776) (end 122.4534 74.803) (width 0.25) (layer B.Cu) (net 4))
 (segment (start 122.428 70.7898) (end 122.428 74.7776) (width 0.25) (layer B.Cu) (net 4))
 (segment (start 130.1496 82.4992) (end 122.4534 74.803) (width 0.25) (layer B.Cu) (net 4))
 (segment (start 133.985 82.4992) (end 130.1496 82.4992) (width 0.25) (layer B.Cu) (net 4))
 (segment (start 149.9616 60.6298) (end 149.8854 60.706) (width 0.25) (layer F.Cu) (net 4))
 (segment (start 149.9616 58.9026) (end 149.9616 60.6298) (width 0.25) (layer F.Cu) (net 4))
 (segment (start 115.998 68.8848) (end 116.0018 68.881) (width 0.5) (layer F.Cu) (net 5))
 (segment (start 112.6998 68.8848) (end 115.998 68.8848) (width 0.5) (layer F.Cu) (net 5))
 (segment (start 123.1176 68.881) (end 123.1392 68.8594) (width 0.5) (layer F.Cu) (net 5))
 (segment (start 116.0018 68.881) (end 123.1176 68.881) (width 0.5) (layer F.Cu) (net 5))
 (segment (start 128.8034 68.8594) (end 128.8288 68.834) (width 0.5) (layer F.Cu) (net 6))
 (segment (start 125.9392 68.8594) (end 128.8034 68.8594) (width 0.5) (layer F.Cu) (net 6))
 (segment (start 125.9646 75.7465) (end 125.9863 75.7682) (width 0.25) (layer F.Cu) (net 6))
 (segment (start 125.9392 75.7211) (end 125.9863 75.7682) (width 0.25) (layer F.Cu) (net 6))
 (segment (start 125.9392 68.8594) (end 125.9392 75.7211) (width 0.25) (layer F.Cu) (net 6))
 (segment (start 112.6998 63.754) (end 116.0018 63.754) (width 0.5) (layer F.Cu) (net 7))
 (segment (start 116.0018 63.754) (end 123.1078 63.754) (width 0.5) (layer F.Cu) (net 7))
 (segment (start 154.8118 62.3824) (end 160.3779 62.3824) (width 0.25) (layer F.Cu) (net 12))
 (segment (start 161.40291 61.35739) (end 160.3779 62.3824) (width 0.25) (layer F.Cu) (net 12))
 (segment (start 167.19919 61.35739) (end 161.40291 61.35739) (width 0.25) (layer F.Cu) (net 12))
 (segment (start 168.3004 62.4586) (end 167.19919 61.35739) (width 0.25) (layer F.Cu) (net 12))
 (segment (start 163.2242 62.3824) (end 168.3004 67.4586) (width 0.25) (layer F.Cu) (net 13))
 (segment (start 162.2529 62.3824) (end 163.2242 62.3824) (width 0.25) (layer F.Cu) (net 13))
 (segment (start 162.2529 66.4111) (end 168.3004 72.4586) (width 0.25) (layer F.Cu) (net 14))
 (segment (start 162.2529 64.4652) (end 162.2529 66.4111) (width 0.25) (layer F.Cu) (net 14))
 (segment (start 127.8613 75.7682) (end 127.8613 77.8002) (width 0.25) (layer F.Cu) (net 15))
 (segment (start 125.9886 77.8025) (end 125.9863 77.8002) (width 0.25) (layer F.Cu) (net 16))
 (segment (start 125.9886 79.8576) (end 125.9886 77.8025) (width 0.25) (layer F.Cu) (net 16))
 (segment (start 127.8636 81.9381) (end 127.8613 81.9404) (width 0.25) (layer F.Cu) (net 17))
 (segment (start 127.8636 79.8576) (end 127.8636 81.9381) (width 0.25) (layer F.Cu) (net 17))
 (segment (start 125.9863 81.9404) (end 124.303 81.9404) (width 0.25) (layer F.Cu) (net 18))
 (segment (start 128.34064 82.96541) (end 127.01131 82.96541) (width 0.25) (layer F.Cu) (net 18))
 (segment (start 127.01131 82.96541) (end 125.9863 81.9404) (width 0.25) (layer F.Cu) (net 18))
 (segment (start 130.07685 81.2292) (end 129.973525 81.332525) (width 0.25) (layer F.Cu) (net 18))
 (segment (start 136.1582 81.2292) (end 130.07685 81.2292) (width 0.25) (layer F.Cu) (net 18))
 (segment (start 128.34064 82.96541) (end 129.973525 81.332525) (width 0.25) (layer F.Cu) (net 18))
 (segment (start 122.4326 81.9358) (end 122.428 81.9404) (width 0.25) (layer F.Cu) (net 19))
 (segment (start 122.4326 79.8322) (end 122.4326 81.9358) (width 0.25) (layer F.Cu) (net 19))
 (segment (start 124.3053 79.8299) (end 124.3076 79.8322) (width 0.25) (layer F.Cu) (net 20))
 (segment (start 124.3053 77.7748) (end 124.3053 79.8299) (width 0.25) (layer F.Cu) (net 20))
 (segment (start 136.1582 78.6892) (end 136.1582 79.9592) (width 0.25) (layer F.Cu) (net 21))
 (segment (start 136.1717 78.6757) (end 136.1582 78.6892) (width 0.25) (layer F.Cu) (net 21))
 (segment (start 136.1717 76.5048) (end 136.1717 78.6757) (width 0.25) (layer F.Cu) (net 21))
 (segment (start 143.6878 81.8619) (end 143.6624 81.8365) (width 0.25) (layer F.Cu) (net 22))
 (segment (start 145.8214 81.8619) (end 143.6878 81.8619) (width 0.25) (layer F.Cu) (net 22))
 (via (at 150.114 65.151) (size 0.8) (drill 0.4) (layers F.Cu B.Cu) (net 22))
 (segment (start 145.8214 81.8619) (end 146.8097 80.8736) (width 0.25) (layer F.Cu) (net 22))
 (segment (start 150.114 65.151) (end 148.5404 65.151) (width 0.25) (layer F.Cu) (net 22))
 (segment (start 148.5404 65.151) (end 148.3118 64.9224) (width 0.25) (layer F.Cu) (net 22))
 (via (at 150.1648 79.2226) (size 0.8) (drill 0.4) (layers F.Cu B.Cu) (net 22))
 (segment (start 146.88389 80.79941) (end 146.8097 80.8736) (width 0.25) (layer F.Cu) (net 22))
 (segment (start 150.114 79.1718) (end 150.1648 79.2226) (width 0.25) (layer B.Cu) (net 22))
 (segment (start 150.114 65.151) (end 150.114 79.1718) (width 0.25) (layer B.Cu) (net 22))
 (segment (start 150.1648 79.9084) (end 149.27379 80.79941) (width 0.25) (layer F.Cu) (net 22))
 (segment (start 150.1648 79.2226) (end 150.1648 79.9084) (width 0.25) (layer F.Cu) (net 22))
 (segment (start 149.27379 80.79941) (end 146.88389 80.79941) (width 0.25) (layer F.Cu) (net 22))
 (segment (start 147.0939 82.7992) (end 148.0312 81.8619) (width 0.25) (layer F.Cu) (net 23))
 (segment (start 141.4082 82.7992) (end 147.0939 82.7992) (width 0.25) (layer F.Cu) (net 23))
 (segment (start 141.1082 82.4992) (end 141.4082 82.7992) (width 0.25) (layer F.Cu) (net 23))
 (segment (start 154.8118 64.9224) (end 158.242 64.9224) (width 0.25) (layer F.Cu) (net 23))
 (via (at 158.242 64.9224) (size 0.8) (drill 0.4) (layers F.Cu B.Cu) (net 23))
 (segment (start 148.2067 81.6864) (end 148.0312 81.8619) (width 0.25) (layer F.Cu) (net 23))
 (via (at 150.114 81.8619) (size 0.8) (drill 0.4) (layers F.Cu B.Cu) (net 23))
 (segment (start 148.0312 81.8619) (end 150.114 81.8619) (width 0.25) (layer F.Cu) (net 23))
 (segment (start 158.242 73.7339) (end 158.242 64.9224) (width 0.25) (layer B.Cu) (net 23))
 (segment (start 150.114 81.8619) (end 158.242 73.7339) (width 0.25) (layer B.Cu) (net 23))
 (segment (start 154.8118 66.1924) (end 154.8118 66.2166) (width 0.25) (layer F.Cu) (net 24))
 (segment (start 155.83681 66.51741) (end 155.5118 66.1924) (width 0.25) (layer F.Cu) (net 24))
 (segment (start 155.83681 77.20819) (end 155.83681 66.51741) (width 0.25) (layer F.Cu) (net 24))
 (segment (start 155.5118 66.1924) (end 154.8118 66.1924) (width 0.25) (layer F.Cu) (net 24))
 (segment (start 138.0213 84.455) (end 148.59 84.455) (width 0.25) (layer F.Cu) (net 24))
 (segment (start 148.59 84.455) (end 155.83681 77.20819) (width 0.25) (layer F.Cu) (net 24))
 (segment (start 159.5651 63.6524) (end 160.3779 64.4652) (width 0.25) (layer F.Cu) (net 25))
 (segment (start 154.8118 63.6524) (end 159.5651 63.6524) (width 0.25) (layer F.Cu) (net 25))
 (segment (start 138.9888 68.834) (end 138.9888 72.517) (width 0.5) (layer F.Cu) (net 26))
 (segment (start 147.286799 65.867399) (end 147.6118 66.1924) (width 0.25) (layer F.Cu) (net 27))
 (segment (start 148.3118 62.3824) (end 147.955 62.3824) (width 0.25) (layer F.Cu) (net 27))
 (segment (start 147.6118 66.1924) (end 148.3118 66.1924) (width 0.25) (layer F.Cu) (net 27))
 (segment (start 147.286799 63.050601) (end 147.286799 65.867399) (width 0.25) (layer F.Cu) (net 27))
 (segment (start 147.955 62.3824) (end 147.286799 63.050601) (width 0.25) (layer F.Cu) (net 27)))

